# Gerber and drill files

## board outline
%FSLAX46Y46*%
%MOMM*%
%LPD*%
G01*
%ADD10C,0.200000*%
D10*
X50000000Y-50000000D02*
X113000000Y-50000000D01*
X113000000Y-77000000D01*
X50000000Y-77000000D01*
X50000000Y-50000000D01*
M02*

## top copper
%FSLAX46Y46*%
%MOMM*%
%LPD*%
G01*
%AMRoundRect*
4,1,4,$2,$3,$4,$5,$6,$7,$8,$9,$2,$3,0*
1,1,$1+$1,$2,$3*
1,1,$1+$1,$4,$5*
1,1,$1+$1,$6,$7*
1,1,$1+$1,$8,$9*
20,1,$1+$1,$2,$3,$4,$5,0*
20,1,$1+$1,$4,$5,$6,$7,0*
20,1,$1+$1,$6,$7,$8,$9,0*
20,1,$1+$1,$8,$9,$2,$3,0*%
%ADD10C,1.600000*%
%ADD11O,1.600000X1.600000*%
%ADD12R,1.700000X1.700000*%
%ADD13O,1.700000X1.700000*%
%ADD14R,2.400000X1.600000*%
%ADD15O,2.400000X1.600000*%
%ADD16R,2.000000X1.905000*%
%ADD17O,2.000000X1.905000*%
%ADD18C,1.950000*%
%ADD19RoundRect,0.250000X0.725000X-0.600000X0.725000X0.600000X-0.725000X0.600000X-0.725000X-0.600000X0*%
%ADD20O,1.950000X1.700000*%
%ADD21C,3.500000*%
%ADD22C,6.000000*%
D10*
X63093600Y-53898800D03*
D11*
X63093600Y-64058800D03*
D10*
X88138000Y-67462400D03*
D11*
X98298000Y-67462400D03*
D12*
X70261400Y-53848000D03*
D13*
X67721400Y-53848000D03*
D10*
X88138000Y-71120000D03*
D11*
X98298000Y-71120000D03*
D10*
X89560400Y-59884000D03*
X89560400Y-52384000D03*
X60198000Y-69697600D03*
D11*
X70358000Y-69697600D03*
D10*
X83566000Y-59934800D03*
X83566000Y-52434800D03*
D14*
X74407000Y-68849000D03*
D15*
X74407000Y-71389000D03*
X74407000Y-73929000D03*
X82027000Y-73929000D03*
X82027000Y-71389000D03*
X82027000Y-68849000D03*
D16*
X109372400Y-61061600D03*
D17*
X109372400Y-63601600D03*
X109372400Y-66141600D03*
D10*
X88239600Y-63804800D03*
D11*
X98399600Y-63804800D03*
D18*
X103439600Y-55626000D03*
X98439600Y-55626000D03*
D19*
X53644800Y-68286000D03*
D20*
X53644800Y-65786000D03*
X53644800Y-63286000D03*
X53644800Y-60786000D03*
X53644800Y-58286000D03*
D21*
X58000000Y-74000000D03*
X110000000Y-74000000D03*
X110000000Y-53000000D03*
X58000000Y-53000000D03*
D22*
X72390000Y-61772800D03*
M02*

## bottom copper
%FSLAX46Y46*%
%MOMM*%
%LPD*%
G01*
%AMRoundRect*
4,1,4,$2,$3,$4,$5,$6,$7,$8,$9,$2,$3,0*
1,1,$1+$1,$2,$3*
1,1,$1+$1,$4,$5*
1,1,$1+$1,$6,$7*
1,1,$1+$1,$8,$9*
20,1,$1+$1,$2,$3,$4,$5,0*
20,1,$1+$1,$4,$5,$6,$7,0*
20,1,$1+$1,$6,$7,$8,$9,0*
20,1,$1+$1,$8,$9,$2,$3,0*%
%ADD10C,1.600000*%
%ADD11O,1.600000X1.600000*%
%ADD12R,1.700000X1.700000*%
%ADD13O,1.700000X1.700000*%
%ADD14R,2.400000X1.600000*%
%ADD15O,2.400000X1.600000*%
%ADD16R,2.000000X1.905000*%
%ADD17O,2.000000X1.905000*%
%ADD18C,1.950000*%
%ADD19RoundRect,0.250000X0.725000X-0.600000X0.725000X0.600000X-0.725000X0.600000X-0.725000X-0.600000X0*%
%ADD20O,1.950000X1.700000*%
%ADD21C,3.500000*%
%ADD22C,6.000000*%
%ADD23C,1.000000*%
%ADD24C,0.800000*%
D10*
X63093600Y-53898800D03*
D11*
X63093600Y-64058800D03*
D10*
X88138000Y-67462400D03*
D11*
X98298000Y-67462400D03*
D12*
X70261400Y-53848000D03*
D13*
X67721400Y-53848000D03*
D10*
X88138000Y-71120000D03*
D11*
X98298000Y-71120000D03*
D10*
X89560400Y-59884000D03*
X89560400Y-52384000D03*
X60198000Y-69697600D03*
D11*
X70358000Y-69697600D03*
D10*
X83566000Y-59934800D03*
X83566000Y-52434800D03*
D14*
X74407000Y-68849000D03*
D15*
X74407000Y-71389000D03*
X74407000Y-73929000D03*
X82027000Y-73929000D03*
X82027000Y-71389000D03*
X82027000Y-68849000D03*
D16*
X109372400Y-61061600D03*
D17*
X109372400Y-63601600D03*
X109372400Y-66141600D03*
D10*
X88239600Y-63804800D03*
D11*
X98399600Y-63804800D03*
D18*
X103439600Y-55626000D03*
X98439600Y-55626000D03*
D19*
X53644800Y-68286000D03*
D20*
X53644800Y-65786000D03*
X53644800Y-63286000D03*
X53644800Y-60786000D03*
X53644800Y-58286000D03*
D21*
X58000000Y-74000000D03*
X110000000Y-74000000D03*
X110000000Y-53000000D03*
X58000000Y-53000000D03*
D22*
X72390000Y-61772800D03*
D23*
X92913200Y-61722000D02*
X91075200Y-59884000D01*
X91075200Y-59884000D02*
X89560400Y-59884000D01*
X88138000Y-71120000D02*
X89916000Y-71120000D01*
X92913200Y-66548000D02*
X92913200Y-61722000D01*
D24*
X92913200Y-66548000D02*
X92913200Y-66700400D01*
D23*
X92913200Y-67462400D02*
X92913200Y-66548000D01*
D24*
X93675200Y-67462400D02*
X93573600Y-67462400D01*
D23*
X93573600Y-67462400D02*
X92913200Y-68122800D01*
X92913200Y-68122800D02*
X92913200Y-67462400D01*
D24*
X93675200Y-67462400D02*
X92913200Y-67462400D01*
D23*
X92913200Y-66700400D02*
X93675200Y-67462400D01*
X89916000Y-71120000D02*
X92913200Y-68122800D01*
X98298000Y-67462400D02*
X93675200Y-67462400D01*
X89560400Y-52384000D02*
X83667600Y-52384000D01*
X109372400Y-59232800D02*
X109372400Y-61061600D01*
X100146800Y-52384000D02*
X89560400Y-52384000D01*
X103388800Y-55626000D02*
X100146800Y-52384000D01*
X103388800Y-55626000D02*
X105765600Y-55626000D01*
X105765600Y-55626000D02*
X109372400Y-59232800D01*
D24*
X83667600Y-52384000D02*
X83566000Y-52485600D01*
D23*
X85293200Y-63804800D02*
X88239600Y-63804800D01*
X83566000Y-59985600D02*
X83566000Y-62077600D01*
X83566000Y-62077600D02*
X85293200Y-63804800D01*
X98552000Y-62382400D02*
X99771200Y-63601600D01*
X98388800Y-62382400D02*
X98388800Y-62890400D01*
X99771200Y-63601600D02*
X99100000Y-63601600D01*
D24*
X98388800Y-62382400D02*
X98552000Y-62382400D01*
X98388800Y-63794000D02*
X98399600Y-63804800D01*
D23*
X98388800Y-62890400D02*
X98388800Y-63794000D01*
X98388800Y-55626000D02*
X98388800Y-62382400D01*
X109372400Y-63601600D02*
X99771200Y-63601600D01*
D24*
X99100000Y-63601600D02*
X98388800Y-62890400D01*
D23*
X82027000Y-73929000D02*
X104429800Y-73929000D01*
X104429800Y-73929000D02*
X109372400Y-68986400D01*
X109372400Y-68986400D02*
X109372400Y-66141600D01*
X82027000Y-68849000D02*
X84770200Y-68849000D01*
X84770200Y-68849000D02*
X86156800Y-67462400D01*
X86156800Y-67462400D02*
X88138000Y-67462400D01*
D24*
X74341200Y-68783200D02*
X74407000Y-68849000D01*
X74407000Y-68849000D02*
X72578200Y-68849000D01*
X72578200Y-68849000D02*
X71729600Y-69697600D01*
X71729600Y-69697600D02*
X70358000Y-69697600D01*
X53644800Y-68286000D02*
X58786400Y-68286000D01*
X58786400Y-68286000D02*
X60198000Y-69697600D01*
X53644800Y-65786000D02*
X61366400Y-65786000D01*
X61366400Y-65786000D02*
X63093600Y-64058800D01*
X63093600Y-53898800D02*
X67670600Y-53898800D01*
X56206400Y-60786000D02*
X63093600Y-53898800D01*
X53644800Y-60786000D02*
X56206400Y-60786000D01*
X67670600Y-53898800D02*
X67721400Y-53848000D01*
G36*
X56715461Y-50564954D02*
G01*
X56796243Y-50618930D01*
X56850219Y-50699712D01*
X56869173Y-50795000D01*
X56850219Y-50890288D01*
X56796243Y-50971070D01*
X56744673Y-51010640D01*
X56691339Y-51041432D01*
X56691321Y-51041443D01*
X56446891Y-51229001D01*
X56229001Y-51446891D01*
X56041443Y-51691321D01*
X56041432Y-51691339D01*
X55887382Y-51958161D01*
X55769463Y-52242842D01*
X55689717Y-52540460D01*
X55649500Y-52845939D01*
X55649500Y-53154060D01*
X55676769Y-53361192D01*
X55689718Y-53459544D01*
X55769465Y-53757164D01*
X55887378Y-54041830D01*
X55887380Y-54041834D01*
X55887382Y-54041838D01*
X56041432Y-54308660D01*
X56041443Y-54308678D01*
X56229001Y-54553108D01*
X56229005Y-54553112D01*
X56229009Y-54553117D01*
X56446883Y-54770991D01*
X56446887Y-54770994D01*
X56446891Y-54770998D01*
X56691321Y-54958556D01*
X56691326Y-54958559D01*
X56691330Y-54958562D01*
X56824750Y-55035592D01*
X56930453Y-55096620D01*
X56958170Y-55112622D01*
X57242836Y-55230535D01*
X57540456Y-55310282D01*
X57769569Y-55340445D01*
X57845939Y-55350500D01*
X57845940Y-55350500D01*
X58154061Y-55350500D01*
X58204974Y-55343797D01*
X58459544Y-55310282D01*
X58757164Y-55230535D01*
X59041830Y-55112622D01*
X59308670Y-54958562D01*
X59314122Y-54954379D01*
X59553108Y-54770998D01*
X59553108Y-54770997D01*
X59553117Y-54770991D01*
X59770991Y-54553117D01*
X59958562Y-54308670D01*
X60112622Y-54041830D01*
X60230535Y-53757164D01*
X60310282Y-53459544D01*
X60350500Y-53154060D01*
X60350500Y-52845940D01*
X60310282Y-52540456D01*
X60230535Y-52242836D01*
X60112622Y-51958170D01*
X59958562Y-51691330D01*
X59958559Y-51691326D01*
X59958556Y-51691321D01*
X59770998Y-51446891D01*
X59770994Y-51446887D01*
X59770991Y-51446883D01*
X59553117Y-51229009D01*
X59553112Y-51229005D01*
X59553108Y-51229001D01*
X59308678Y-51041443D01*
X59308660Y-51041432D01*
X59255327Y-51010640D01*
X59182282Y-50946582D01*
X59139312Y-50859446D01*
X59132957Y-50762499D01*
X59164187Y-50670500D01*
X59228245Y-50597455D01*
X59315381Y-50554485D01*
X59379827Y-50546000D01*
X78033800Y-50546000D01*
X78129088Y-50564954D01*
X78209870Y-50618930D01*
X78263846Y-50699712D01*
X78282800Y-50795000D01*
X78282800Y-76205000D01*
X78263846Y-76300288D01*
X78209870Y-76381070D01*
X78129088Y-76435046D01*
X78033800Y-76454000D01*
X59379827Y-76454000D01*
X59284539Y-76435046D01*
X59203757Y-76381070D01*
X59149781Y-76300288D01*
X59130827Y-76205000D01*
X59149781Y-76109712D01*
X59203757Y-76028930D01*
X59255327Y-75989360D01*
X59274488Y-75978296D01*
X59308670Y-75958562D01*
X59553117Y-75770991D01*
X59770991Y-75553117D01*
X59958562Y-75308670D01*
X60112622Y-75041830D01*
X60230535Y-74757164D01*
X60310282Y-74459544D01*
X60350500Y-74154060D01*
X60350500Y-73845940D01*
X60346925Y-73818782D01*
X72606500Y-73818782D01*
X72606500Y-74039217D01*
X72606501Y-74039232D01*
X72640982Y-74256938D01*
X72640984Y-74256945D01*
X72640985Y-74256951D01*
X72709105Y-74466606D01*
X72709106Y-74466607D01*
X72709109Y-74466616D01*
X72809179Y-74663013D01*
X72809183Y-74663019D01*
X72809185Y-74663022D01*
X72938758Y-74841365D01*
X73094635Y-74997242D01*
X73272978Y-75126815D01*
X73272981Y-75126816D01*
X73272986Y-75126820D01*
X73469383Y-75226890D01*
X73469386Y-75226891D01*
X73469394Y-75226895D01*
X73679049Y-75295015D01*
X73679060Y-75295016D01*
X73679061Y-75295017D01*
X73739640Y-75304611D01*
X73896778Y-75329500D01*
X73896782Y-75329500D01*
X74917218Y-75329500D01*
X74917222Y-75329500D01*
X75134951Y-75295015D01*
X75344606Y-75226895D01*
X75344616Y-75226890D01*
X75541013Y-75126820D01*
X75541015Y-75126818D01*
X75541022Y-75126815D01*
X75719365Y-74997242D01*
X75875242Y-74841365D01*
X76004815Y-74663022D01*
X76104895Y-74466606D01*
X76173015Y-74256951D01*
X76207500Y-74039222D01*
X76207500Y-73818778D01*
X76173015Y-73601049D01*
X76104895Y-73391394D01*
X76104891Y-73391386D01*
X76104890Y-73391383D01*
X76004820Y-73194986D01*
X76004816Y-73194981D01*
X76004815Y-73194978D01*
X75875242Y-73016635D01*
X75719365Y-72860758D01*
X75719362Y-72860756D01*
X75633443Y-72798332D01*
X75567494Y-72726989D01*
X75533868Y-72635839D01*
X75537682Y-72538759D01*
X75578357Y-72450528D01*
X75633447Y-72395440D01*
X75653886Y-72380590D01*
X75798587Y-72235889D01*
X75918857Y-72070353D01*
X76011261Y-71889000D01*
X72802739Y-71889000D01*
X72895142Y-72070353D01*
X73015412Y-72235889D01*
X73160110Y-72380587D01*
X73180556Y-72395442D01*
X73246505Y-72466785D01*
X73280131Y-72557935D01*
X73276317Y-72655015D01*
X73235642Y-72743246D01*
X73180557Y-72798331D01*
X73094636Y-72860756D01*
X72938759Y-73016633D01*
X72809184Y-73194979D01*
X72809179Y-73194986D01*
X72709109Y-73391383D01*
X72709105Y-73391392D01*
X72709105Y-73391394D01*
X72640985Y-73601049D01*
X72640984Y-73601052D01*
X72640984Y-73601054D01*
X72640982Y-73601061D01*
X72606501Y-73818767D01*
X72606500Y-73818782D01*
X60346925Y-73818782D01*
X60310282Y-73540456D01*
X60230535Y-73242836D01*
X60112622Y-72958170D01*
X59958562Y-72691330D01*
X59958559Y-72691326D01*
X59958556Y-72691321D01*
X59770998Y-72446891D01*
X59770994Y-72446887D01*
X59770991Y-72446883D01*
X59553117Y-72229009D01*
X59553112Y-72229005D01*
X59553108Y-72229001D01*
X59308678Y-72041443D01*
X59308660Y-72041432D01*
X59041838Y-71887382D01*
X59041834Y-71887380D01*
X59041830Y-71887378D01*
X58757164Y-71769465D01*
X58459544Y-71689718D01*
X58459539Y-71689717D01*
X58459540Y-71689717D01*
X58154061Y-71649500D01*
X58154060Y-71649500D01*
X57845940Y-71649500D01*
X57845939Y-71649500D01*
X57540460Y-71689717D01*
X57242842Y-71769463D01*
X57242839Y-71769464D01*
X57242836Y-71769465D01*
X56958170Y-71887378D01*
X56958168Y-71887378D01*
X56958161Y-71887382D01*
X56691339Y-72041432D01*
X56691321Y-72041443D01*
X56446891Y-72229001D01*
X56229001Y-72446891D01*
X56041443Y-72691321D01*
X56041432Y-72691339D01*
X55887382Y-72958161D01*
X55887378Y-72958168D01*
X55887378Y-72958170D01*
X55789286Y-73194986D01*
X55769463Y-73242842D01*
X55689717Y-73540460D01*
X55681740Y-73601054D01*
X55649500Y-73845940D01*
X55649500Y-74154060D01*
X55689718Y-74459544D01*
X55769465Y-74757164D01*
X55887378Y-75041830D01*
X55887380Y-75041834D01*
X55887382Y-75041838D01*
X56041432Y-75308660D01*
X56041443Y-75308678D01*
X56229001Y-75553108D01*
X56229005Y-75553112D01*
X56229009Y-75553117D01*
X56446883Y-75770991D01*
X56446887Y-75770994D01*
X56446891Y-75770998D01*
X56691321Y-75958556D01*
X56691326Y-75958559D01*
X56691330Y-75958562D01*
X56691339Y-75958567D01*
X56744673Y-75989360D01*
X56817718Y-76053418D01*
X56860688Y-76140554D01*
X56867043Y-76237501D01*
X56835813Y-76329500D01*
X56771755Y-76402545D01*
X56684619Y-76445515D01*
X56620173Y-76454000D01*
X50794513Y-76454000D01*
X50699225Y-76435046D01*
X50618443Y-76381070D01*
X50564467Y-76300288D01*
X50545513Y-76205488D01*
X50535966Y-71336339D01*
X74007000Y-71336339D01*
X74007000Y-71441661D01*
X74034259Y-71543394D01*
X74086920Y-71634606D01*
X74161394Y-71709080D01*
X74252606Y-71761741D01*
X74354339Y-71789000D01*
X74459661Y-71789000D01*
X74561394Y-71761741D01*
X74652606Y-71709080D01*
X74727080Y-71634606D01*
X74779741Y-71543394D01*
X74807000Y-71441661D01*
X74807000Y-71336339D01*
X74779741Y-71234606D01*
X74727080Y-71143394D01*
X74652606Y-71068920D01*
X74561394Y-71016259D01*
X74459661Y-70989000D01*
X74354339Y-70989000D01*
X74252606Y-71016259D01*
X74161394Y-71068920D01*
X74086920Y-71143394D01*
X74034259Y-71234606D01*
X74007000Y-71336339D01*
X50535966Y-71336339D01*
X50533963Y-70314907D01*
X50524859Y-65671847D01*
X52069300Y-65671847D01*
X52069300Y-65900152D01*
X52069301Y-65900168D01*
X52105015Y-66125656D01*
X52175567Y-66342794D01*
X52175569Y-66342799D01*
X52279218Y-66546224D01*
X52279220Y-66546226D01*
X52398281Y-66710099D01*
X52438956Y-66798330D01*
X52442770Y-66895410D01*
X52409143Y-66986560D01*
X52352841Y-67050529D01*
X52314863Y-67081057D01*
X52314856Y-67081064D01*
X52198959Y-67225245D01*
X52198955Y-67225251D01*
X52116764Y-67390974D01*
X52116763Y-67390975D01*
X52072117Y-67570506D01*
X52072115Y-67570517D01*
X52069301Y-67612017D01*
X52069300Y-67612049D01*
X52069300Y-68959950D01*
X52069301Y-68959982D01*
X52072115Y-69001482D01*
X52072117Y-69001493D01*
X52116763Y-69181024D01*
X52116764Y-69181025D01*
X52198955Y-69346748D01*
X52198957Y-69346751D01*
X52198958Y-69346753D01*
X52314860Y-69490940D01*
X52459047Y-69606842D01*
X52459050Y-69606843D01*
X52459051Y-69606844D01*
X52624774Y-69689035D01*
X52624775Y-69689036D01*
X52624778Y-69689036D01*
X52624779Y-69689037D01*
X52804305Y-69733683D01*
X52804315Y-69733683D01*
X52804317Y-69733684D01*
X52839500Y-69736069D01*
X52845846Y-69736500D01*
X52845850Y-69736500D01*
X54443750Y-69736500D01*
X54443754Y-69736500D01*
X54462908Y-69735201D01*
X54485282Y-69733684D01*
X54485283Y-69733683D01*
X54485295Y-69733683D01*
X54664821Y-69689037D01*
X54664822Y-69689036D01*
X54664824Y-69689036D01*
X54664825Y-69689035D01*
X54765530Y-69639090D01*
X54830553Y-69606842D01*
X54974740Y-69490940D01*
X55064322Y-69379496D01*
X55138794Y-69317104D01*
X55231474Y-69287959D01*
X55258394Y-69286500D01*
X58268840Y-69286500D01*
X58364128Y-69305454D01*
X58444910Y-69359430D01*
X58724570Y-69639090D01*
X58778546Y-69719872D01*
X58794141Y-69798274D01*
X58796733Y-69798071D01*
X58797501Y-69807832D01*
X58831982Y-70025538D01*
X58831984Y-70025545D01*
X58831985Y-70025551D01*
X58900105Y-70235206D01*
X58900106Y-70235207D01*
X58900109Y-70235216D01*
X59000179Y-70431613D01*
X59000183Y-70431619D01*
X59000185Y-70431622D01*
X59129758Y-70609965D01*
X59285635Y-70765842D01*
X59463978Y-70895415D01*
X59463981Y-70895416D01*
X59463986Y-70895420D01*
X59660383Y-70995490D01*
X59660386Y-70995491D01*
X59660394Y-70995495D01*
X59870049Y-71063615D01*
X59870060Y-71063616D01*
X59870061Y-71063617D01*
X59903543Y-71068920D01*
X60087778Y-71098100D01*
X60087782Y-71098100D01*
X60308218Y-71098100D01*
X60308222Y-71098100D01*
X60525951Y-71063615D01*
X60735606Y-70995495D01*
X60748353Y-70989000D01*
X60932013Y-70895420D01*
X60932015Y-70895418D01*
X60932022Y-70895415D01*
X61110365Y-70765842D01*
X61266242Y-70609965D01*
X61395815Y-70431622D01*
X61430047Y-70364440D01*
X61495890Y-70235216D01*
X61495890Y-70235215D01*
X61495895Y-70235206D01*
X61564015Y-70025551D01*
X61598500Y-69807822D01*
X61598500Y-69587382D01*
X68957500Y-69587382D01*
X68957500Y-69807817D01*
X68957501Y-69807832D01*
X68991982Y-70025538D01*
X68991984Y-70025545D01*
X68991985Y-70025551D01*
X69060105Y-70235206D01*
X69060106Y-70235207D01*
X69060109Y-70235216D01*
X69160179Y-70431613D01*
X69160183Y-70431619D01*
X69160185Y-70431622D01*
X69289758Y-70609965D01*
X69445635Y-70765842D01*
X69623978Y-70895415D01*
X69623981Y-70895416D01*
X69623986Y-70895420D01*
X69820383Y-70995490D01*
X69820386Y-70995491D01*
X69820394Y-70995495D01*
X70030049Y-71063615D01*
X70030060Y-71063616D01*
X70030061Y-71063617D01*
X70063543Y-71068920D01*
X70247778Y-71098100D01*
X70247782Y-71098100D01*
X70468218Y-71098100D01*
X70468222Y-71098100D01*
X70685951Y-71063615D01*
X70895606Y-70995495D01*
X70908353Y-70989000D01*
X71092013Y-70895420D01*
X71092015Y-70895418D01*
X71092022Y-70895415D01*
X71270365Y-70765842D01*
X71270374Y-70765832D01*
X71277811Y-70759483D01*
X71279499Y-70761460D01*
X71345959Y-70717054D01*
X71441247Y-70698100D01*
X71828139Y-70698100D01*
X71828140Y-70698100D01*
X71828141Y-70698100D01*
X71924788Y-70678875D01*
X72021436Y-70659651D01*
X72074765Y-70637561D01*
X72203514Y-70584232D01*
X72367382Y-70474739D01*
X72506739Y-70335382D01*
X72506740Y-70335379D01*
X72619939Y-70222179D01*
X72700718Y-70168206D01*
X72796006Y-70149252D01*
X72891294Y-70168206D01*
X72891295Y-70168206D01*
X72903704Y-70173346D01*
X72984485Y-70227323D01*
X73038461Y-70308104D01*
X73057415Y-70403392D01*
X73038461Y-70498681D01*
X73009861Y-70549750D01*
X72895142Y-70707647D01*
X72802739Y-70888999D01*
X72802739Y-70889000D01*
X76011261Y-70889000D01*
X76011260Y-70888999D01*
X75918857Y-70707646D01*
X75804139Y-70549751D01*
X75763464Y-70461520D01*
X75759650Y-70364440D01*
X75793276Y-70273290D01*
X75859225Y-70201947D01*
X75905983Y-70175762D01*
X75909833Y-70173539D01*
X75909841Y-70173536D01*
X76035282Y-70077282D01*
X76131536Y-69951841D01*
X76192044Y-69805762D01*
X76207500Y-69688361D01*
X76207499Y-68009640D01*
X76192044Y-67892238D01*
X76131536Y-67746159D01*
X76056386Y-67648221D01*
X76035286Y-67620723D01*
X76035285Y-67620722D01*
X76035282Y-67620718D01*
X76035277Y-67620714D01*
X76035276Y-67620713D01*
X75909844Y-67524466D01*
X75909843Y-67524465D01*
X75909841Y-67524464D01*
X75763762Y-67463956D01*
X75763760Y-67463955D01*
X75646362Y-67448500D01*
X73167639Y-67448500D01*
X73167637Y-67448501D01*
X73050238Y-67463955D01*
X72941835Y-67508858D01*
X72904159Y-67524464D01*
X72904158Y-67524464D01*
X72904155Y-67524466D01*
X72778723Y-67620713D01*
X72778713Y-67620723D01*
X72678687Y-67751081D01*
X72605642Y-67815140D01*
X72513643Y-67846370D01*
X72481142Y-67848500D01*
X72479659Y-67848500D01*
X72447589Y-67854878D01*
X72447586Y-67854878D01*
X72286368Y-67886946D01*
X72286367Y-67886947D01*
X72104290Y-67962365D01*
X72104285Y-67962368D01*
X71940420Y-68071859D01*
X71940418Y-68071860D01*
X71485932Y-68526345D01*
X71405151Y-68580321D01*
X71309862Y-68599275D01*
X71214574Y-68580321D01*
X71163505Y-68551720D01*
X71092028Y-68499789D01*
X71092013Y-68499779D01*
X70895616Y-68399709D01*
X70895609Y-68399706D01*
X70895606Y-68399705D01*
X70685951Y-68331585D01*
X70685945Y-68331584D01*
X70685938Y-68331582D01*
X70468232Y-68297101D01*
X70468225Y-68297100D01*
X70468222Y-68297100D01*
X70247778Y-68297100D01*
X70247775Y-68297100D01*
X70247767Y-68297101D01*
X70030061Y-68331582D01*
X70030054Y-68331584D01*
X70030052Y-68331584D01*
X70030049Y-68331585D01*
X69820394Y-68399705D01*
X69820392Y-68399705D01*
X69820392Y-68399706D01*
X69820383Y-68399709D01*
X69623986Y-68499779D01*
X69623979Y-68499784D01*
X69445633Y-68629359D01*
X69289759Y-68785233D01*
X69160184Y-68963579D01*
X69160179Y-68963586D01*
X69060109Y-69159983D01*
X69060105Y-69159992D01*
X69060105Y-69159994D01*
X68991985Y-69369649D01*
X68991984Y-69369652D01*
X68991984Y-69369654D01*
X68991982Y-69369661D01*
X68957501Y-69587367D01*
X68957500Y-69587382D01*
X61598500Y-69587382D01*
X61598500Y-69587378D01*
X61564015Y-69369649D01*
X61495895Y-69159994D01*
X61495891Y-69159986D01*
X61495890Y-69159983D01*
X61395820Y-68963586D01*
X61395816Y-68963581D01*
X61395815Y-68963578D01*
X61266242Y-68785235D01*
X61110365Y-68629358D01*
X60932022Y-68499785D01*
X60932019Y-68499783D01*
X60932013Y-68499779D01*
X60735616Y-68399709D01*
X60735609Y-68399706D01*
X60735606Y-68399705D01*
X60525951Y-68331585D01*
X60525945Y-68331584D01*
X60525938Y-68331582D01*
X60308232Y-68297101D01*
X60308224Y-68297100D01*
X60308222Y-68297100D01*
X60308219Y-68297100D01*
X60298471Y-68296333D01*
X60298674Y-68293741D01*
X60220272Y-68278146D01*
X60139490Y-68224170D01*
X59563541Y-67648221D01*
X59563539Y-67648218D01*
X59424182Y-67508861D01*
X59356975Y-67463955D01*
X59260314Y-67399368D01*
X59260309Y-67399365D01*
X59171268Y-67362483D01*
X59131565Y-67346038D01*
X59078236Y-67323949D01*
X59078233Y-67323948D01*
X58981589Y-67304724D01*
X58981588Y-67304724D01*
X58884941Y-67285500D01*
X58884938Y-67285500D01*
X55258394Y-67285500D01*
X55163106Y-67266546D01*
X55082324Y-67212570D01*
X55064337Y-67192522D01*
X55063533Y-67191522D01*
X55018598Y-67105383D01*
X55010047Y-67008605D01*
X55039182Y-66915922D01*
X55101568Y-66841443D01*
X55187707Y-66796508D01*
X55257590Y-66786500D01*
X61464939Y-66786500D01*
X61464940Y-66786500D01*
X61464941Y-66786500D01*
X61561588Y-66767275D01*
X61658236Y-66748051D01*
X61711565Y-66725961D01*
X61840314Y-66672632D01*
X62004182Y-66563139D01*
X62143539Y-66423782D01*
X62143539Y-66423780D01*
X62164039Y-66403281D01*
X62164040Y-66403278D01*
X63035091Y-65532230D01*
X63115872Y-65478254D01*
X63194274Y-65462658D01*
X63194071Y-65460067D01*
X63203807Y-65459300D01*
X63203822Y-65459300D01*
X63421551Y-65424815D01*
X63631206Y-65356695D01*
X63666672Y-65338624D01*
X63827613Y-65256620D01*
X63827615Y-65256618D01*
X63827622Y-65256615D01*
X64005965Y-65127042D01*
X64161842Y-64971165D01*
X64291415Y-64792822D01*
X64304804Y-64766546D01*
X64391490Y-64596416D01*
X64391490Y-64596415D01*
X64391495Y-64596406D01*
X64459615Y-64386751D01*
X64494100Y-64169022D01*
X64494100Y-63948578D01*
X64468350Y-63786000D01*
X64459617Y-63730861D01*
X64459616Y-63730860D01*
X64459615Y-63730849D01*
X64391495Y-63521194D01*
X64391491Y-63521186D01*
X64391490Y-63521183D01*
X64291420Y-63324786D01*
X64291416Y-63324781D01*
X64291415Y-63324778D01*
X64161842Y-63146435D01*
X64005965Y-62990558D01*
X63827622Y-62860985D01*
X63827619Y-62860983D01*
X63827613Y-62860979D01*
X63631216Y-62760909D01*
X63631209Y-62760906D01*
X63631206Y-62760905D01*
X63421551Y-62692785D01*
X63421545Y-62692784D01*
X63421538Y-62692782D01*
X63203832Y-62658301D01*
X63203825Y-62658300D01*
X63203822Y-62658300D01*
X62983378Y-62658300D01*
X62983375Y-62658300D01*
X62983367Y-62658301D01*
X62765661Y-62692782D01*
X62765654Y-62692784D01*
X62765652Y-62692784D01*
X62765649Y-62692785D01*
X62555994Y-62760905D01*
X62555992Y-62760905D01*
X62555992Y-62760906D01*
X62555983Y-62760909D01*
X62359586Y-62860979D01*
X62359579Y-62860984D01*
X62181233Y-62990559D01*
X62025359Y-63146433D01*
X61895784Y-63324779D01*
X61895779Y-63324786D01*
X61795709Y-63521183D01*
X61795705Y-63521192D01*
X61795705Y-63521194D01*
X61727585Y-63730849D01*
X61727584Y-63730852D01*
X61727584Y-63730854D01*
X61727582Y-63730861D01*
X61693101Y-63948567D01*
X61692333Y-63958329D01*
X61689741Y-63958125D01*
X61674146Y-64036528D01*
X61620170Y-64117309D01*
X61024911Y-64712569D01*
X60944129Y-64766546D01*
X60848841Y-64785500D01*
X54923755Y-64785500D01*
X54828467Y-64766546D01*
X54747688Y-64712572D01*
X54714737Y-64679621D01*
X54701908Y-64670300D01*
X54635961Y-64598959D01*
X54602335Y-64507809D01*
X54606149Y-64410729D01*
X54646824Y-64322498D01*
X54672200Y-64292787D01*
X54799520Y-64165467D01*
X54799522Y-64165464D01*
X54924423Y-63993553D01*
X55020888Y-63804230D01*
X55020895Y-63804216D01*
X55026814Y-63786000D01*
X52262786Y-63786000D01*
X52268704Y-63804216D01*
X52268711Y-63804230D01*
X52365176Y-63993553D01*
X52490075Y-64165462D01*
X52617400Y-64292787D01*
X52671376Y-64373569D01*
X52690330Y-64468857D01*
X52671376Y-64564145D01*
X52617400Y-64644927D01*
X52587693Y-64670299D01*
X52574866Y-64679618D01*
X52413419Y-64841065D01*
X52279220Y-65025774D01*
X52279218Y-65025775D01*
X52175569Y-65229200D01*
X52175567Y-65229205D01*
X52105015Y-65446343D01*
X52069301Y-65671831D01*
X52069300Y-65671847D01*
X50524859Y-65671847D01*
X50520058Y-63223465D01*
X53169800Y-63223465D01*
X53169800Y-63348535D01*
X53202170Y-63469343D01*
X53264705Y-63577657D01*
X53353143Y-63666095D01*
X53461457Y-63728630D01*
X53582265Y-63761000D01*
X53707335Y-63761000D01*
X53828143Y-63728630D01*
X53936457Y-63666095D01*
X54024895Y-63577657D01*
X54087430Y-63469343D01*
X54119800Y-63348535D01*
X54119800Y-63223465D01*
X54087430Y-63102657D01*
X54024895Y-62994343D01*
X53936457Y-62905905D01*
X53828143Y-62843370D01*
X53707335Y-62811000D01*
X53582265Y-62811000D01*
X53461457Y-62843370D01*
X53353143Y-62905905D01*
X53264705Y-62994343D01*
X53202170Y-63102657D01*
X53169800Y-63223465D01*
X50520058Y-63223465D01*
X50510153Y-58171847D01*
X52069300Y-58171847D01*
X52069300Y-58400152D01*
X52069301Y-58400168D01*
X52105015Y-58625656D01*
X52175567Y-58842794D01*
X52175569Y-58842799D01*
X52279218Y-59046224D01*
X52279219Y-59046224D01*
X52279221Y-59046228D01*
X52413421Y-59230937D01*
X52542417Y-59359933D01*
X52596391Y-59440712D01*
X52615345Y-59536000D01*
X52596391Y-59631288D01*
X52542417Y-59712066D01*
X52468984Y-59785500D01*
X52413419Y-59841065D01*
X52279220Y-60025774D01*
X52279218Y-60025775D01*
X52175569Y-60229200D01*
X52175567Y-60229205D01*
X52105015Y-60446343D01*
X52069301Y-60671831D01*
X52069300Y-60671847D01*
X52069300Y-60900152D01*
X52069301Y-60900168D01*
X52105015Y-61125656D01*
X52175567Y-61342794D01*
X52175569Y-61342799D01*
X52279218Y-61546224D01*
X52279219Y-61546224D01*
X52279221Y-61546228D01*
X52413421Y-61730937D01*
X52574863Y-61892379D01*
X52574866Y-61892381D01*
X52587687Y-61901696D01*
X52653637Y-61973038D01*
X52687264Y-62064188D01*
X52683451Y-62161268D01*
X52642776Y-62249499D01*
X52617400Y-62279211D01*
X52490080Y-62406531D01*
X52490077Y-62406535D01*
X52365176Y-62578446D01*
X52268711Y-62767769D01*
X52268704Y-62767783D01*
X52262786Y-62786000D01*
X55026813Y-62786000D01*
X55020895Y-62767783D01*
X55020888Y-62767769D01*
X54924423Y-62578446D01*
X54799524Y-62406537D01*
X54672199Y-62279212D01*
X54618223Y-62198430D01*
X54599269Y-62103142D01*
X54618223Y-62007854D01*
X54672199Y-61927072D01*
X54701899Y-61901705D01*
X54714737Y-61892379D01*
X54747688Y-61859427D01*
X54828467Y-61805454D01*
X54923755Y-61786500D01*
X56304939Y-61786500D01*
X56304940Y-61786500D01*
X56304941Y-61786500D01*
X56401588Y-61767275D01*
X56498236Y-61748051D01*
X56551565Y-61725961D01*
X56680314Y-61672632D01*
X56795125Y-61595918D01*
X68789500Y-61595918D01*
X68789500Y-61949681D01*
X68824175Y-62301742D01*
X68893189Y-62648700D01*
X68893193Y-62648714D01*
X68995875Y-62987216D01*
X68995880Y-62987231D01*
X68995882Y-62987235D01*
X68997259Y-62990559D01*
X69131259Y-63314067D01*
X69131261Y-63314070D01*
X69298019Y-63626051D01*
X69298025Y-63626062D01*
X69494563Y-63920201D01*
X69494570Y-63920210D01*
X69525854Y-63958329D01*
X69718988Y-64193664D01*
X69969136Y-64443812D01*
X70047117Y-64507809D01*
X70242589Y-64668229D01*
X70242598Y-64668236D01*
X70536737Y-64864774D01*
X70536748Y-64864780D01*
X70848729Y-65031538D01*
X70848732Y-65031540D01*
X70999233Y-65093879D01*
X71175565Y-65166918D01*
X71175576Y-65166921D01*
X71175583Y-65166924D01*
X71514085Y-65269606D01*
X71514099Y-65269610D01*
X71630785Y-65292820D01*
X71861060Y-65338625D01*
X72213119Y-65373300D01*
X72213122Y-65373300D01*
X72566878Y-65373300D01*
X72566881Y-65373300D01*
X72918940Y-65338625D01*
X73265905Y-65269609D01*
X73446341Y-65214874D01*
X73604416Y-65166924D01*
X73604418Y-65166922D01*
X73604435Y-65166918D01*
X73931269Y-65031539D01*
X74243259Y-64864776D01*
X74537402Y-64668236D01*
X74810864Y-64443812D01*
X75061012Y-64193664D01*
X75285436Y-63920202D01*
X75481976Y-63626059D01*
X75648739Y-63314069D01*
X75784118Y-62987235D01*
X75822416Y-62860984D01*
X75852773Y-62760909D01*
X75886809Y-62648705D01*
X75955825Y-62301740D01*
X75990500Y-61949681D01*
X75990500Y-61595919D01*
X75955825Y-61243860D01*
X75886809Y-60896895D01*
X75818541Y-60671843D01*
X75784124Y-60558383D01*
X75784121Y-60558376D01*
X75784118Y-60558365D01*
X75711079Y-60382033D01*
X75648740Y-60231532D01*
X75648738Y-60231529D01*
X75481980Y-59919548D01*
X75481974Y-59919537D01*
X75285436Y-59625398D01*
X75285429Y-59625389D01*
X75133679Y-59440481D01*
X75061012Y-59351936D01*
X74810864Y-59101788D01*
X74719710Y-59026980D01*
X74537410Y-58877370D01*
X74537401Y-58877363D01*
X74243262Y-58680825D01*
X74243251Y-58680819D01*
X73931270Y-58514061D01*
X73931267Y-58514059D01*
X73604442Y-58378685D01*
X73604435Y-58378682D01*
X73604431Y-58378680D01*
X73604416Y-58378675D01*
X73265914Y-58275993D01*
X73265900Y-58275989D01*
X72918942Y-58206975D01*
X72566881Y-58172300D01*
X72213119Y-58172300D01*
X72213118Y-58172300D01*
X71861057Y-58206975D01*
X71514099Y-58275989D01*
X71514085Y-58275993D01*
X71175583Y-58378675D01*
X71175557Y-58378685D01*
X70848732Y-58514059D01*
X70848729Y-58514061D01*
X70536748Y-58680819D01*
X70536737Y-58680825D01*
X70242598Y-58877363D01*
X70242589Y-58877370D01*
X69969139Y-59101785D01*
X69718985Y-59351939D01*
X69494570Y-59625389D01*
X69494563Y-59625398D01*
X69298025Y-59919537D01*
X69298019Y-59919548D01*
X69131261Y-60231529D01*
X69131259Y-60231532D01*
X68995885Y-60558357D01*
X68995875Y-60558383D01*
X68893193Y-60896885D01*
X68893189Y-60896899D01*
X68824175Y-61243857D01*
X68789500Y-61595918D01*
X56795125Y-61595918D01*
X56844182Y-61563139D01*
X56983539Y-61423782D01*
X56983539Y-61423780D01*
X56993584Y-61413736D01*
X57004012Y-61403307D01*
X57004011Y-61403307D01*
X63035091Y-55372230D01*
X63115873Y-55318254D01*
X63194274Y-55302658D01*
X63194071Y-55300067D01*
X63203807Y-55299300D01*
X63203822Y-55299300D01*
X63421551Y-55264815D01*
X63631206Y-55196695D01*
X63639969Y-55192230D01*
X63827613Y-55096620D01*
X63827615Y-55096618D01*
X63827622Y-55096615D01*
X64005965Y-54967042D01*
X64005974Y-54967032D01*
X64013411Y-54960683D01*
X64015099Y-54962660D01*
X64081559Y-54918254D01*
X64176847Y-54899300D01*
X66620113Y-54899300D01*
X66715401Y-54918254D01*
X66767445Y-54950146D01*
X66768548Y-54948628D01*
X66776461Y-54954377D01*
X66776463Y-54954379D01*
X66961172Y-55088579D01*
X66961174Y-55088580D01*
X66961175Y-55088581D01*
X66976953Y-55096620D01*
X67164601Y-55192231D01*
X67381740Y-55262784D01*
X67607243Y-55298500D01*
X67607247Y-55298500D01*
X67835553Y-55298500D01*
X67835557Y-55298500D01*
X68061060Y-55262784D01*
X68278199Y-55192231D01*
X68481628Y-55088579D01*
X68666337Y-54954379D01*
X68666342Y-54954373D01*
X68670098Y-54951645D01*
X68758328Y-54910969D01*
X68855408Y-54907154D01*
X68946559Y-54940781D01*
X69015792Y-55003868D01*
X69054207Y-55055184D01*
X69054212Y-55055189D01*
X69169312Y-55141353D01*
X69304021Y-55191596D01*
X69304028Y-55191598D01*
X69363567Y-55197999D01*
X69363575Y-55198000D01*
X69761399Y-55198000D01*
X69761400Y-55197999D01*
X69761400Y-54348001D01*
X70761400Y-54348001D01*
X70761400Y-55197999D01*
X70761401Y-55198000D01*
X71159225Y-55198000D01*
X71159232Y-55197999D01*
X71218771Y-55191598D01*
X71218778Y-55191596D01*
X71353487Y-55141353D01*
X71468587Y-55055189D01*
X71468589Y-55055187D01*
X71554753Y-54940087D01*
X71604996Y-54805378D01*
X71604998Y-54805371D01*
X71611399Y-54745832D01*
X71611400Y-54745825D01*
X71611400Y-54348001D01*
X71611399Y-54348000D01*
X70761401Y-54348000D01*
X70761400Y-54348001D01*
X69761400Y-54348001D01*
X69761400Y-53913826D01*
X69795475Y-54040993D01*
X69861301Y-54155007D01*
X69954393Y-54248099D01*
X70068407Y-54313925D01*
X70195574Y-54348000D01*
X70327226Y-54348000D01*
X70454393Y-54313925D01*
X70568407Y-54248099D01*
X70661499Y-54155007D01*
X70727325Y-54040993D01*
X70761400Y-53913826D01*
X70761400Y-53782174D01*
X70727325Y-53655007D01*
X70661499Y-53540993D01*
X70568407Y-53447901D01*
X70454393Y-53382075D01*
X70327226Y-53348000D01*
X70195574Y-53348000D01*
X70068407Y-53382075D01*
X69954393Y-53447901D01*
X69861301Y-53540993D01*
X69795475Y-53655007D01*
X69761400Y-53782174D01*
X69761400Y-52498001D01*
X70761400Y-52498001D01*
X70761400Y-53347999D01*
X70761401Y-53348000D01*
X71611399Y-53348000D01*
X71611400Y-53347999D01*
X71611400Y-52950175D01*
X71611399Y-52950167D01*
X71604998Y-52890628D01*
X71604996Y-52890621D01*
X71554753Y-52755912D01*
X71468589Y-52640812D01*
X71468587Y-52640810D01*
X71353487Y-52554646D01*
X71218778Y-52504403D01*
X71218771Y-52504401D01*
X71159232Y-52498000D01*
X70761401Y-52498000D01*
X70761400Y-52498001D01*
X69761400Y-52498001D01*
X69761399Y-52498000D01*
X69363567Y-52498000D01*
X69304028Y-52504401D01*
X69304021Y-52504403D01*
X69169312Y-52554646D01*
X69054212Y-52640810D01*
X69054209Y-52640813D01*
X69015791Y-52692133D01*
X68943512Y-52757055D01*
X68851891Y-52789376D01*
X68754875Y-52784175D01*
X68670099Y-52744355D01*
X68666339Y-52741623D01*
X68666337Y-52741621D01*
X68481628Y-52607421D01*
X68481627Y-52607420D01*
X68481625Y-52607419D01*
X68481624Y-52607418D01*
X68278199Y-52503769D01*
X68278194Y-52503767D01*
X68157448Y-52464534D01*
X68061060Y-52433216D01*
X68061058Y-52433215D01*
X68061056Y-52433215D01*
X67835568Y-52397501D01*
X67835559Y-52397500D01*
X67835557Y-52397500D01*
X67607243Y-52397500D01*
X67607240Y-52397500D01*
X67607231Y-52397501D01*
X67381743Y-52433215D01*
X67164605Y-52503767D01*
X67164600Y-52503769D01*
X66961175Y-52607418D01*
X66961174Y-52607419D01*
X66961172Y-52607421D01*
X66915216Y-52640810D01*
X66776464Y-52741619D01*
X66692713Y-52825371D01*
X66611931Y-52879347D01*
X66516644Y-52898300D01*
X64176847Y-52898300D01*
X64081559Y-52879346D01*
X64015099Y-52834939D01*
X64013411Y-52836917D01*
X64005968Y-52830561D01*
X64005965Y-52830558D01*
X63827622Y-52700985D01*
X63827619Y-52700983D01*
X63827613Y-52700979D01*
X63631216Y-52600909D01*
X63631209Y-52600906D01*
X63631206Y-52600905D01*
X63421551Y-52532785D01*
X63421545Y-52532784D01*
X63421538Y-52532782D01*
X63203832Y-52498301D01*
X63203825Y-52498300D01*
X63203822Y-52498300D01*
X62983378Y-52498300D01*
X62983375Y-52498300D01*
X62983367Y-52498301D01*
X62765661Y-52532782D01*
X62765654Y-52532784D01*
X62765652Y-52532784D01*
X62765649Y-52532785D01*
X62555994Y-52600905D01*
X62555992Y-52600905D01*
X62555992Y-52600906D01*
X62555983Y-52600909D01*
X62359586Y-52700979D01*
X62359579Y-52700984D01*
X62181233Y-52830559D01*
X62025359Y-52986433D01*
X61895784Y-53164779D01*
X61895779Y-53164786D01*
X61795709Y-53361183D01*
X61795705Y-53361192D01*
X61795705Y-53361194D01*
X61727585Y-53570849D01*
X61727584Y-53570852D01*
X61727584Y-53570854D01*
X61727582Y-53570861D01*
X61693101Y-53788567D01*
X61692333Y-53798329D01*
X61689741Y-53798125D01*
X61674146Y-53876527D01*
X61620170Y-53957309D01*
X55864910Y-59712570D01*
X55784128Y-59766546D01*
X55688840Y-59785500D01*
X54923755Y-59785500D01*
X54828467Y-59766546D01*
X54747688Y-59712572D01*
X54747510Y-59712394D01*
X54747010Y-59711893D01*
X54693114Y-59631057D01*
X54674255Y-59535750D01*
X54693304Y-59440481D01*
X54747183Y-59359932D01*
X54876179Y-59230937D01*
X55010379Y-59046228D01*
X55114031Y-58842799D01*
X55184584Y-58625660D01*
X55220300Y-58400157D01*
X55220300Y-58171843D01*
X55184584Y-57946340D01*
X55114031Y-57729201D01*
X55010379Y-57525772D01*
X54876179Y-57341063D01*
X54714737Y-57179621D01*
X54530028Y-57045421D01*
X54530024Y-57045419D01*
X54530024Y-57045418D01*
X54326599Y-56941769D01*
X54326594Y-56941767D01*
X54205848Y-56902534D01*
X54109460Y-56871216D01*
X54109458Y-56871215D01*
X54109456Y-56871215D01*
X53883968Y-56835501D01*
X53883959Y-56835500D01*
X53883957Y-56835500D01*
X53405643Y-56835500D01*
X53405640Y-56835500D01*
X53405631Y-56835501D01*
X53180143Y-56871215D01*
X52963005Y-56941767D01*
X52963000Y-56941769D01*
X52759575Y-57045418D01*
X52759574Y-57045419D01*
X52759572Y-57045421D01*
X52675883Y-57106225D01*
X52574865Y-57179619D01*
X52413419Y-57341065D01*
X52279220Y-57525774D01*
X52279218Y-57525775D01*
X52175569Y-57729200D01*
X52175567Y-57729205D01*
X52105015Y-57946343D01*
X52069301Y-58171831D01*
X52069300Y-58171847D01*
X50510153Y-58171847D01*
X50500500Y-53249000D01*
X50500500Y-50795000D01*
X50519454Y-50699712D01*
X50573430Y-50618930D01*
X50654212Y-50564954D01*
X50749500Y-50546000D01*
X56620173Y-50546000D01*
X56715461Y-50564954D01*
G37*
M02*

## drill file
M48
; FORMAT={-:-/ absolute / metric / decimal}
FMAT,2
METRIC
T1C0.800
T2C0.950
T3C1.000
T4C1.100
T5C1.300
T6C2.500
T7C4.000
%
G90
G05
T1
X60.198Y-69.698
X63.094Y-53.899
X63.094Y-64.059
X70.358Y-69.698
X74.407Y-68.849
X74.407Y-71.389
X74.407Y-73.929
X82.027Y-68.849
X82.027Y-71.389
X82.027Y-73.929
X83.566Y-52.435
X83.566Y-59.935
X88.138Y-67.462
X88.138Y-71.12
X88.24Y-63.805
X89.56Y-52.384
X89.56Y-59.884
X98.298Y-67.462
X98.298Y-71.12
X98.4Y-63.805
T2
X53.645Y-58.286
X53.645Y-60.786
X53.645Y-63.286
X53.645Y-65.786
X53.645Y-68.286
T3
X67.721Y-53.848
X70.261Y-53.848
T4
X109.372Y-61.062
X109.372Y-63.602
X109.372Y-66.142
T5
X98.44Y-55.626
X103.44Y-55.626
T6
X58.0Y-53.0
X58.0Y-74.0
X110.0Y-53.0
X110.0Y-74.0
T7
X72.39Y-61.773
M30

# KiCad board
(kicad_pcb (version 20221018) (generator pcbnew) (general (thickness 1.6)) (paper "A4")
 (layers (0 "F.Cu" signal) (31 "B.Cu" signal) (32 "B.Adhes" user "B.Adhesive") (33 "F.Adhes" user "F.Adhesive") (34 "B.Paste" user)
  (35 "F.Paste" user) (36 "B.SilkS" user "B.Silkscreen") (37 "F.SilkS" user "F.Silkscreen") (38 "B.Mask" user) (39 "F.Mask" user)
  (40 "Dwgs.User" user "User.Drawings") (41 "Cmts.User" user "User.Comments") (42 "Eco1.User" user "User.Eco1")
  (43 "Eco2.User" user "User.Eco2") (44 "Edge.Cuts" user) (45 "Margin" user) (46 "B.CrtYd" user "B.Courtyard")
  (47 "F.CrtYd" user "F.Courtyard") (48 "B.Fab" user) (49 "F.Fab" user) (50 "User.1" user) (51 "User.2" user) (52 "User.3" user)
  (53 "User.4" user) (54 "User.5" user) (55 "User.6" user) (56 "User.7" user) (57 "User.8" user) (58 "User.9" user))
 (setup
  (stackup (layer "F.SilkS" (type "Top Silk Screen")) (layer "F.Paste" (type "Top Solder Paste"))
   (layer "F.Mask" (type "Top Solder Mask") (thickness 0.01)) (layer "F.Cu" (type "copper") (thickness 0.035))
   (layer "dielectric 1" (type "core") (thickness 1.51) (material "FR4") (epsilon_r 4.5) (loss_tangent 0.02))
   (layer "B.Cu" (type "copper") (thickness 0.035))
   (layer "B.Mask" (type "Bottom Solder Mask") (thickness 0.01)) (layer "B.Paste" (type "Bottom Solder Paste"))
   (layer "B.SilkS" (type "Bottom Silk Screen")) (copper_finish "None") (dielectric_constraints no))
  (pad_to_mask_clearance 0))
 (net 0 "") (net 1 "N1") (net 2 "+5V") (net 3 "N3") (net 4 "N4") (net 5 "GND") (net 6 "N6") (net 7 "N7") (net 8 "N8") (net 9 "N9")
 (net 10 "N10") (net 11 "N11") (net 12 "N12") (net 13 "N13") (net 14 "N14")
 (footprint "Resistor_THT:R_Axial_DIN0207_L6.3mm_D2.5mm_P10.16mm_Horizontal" (layer "F.Cu") (at 63.0936 53.8988 -90)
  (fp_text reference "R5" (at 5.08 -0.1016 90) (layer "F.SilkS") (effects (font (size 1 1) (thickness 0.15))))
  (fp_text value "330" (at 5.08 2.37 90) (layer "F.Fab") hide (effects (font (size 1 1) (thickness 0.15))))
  (pad "1" thru_hole circle (at 0 0 270) (size 1.6 1.6) (drill 0.8) (layers "*.Cu" "*.Mask") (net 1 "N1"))
  (pad "2" thru_hole oval (at 10.16 0 270) (size 1.6 1.6) (drill 0.8) (layers "*.Cu" "*.Mask") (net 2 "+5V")))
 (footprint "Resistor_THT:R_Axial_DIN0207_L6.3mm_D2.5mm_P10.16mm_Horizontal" (layer "F.Cu") (at 88.138 67.4624)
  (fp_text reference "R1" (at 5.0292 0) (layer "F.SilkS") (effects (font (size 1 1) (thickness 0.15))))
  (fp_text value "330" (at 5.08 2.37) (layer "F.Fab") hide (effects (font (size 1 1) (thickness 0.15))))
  (pad "1" thru_hole circle (at 0 0) (size 1.6 1.6) (drill 0.8) (layers "*.Cu" "*.Mask") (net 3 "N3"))
  (pad "2" thru_hole oval (at 10.16 0) (size 1.6 1.6) (drill 0.8) (layers "*.Cu" "*.Mask") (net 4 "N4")))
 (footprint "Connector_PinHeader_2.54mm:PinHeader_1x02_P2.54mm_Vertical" (layer "F.Cu") (at 70.2614 53.848 -90)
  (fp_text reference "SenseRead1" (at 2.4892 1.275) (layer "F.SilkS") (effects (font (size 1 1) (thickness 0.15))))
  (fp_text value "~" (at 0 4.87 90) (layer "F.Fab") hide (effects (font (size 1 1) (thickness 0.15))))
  (pad "1" thru_hole rect (at 0 0 270) (size 1.7 1.7) (drill 1) (layers "*.Cu" "*.Mask") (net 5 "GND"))
  (pad "2" thru_hole oval (at 0 2.54 270) (size 1.7 1.7) (drill 1) (layers "*.Cu" "*.Mask") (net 1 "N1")))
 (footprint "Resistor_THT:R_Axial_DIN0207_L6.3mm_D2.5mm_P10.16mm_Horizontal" (layer "F.Cu") (at 88.138 71.12)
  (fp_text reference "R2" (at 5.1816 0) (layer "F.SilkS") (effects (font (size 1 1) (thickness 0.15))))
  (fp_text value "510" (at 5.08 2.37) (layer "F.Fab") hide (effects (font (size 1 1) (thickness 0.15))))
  (pad "1" thru_hole circle (at 0 0) (size 1.6 1.6) (drill 0.8) (layers "*.Cu" "*.Mask") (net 4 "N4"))
  (pad "2" thru_hole oval (at 10.16 0) (size 1.6 1.6) (drill 0.8) (layers "*.Cu" "*.Mask") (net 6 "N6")))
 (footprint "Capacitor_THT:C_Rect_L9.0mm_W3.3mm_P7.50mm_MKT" (layer "F.Cu") (at 89.5604 59.884 90)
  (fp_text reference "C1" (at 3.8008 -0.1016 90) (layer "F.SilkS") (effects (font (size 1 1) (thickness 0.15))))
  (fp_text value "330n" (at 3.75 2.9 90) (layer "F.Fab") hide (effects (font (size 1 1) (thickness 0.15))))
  (pad "1" thru_hole circle (at 0 0 90) (size 1.6 1.6) (drill 0.8) (layers "*.Cu" "*.Mask") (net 4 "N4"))
  (pad "2" thru_hole circle (at 7.5 0 90) (size 1.6 1.6) (drill 0.8) (layers "*.Cu" "*.Mask") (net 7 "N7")))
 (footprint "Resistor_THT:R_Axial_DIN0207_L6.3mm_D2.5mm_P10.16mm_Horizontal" (layer "F.Cu") (at 60.198 69.6976)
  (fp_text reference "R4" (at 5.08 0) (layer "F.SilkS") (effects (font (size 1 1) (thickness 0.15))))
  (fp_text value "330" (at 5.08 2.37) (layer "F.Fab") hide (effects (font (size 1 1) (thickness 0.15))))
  (pad "1" thru_hole circle (at 0 0) (size 1.6 1.6) (drill 0.8) (layers "*.Cu" "*.Mask") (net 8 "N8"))
  (pad "2" thru_hole oval (at 10.16 0) (size 1.6 1.6) (drill 0.8) (layers "*.Cu" "*.Mask") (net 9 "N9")))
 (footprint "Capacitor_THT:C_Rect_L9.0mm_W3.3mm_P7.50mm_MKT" (layer "F.Cu") (at 83.566 59.9348 90)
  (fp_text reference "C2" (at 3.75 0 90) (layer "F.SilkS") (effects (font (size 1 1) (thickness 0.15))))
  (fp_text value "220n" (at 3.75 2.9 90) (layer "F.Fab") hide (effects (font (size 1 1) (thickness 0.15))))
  (pad "1" thru_hole circle (at 0 0 90) (size 1.6 1.6) (drill 0.8) (layers "*.Cu" "*.Mask") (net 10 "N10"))
  (pad "2" thru_hole circle (at 7.5 0 90) (size 1.6 1.6) (drill 0.8) (layers "*.Cu" "*.Mask") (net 7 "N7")))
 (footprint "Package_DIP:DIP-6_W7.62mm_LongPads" (layer "F.Cu") (at 74.407 68.849)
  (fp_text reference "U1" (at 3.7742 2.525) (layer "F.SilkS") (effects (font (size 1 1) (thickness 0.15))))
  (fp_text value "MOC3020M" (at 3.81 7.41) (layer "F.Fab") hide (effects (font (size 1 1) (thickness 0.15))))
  (pad "1" thru_hole rect (at 0 0) (size 2.4 1.6) (drill 0.8) (layers "*.Cu" "*.Mask") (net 9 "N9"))
  (pad "2" thru_hole oval (at 0 2.54) (size 2.4 1.6) (drill 0.8) (layers "*.Cu" "*.Mask") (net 5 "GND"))
  (pad "3" thru_hole oval (at 0 5.08) (size 2.4 1.6) (drill 0.8) (layers "*.Cu" "*.Mask") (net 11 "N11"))
  (pad "4" thru_hole oval (at 7.62 5.08) (size 2.4 1.6) (drill 0.8) (layers "*.Cu" "*.Mask") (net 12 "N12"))
  (pad "5" thru_hole oval (at 7.62 2.54) (size 2.4 1.6) (drill 0.8) (layers "*.Cu" "*.Mask") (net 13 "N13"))
  (pad "6" thru_hole oval (at 7.62 0) (size 2.4 1.6) (drill 0.8) (layers "*.Cu" "*.Mask") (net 3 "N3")))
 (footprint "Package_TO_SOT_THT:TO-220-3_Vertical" (layer "F.Cu") (at 109.3724 61.0616 -90)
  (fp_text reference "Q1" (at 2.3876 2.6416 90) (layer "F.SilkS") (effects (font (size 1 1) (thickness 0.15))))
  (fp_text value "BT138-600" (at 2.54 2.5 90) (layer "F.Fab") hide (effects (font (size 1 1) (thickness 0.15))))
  (pad "1" thru_hole rect (at 0 0 270) (size 1.905 2) (drill 1.1) (layers "*.Cu" "*.Mask") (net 7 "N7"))
  (pad "2" thru_hole oval (at 2.54 0 270) (size 1.905 2) (drill 1.1) (layers "*.Cu" "*.Mask") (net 6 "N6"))
  (pad "3" thru_hole oval (at 5.08 0 270) (size 1.905 2) (drill 1.1) (layers "*.Cu" "*.Mask") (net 12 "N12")))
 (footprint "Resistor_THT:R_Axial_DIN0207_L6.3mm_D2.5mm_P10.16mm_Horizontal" (layer "F.Cu") (at 88.2396 63.8048)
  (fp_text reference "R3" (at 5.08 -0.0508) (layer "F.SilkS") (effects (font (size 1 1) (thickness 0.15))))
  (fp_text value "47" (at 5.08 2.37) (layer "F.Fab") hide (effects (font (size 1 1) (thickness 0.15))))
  (pad "1" thru_hole circle (at 0 0) (size 1.6 1.6) (drill 0.8) (layers "*.Cu" "*.Mask") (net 10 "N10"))
  (pad "2" thru_hole oval (at 10.16 0) (size 1.6 1.6) (drill 0.8) (layers "*.Cu" "*.Mask") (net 6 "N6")))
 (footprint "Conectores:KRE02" (layer "F.Cu") (at 103.4396 55.626 180)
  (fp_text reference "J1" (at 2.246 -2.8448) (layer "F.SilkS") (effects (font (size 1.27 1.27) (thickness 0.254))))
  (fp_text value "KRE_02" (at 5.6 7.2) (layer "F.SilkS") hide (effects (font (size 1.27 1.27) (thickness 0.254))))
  (pad "1" thru_hole circle (at 0 0 180) (size 1.95 1.95) (drill 1.3) (layers "*.Cu" "*.Mask") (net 7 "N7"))
  (pad "2" thru_hole circle (at 5 0 180) (size 1.95 1.95) (drill 1.3) (layers "*.Cu" "*.Mask") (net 6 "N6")))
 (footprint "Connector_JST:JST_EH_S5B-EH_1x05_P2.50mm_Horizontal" (layer "F.Cu") (at 53.6448 68.286 90)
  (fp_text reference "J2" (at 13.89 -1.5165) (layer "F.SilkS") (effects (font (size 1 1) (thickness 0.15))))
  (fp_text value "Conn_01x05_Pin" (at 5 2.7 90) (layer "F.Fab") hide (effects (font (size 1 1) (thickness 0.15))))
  (pad "1" thru_hole roundrect (at 0 0 90) (size 1.7 1.95) (drill 0.95) (layers "*.Cu" "*.Mask") (roundrect_rratio 0.147059) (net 8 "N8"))
  (pad "2" thru_hole oval (at 2.5 0 90) (size 1.7 1.95) (drill 0.95) (layers "*.Cu" "*.Mask") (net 2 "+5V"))
  (pad "3" thru_hole oval (at 5 0 90) (size 1.7 1.95) (drill 0.95) (layers "*.Cu" "*.Mask") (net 5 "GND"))
  (pad "4" thru_hole oval (at 7.5 0 90) (size 1.7 1.95) (drill 0.95) (layers "*.Cu" "*.Mask") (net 1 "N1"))
  (pad "5" thru_hole oval (at 10 0 90) (size 1.7 1.95) (drill 0.95) (layers "*.Cu" "*.Mask") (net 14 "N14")))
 (gr_rect (start 50 50) (end 113 77) (stroke (width 0.2) (type default)) (fill none) (layer "Edge.Cuts"))
 (via (at 58 74) (size 3.5) (drill 2.5) (layers "F.Cu" "B.Cu") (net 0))
 (via (at 110 74) (size 3.5) (drill 2.5) (layers "F.Cu" "B.Cu") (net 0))
 (via (at 110 53) (size 3.5) (drill 2.5) (layers "F.Cu" "B.Cu") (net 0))
 (via (at 58 53) (size 3.5) (drill 2.5) (layers "F.Cu" "B.Cu") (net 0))
 (via (at 72.39 61.7728) (size 6) (drill 4) (layers "F.Cu" "B.Cu") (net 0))
 (segment (start 92.9132 61.722) (end 91.0752 59.884) (width 1) (layer "B.Cu") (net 4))
 (segment (start 91.0752 59.884) (end 89.5604 59.884) (width 1) (layer "B.Cu") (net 4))
 (segment (start 88.138 71.12) (end 89.916 71.12) (width 1) (layer "B.Cu") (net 4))
 (segment (start 92.9132 66.548) (end 92.9132 61.722) (width 1) (layer "B.Cu") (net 4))
 (segment (start 92.9132 66.548) (end 92.9132 66.7004) (width 0.8) (layer "B.Cu") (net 4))
 (segment (start 92.9132 67.4624) (end 92.9132 66.548) (width 1) (layer "B.Cu") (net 4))
 (segment (start 93.6752 67.4624) (end 93.5736 67.4624) (width 0.8) (layer "B.Cu") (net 4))
 (segment (start 93.5736 67.4624) (end 92.9132 68.1228) (width 1) (layer "B.Cu") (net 4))
 (segment (start 92.9132 68.1228) (end 92.9132 67.4624) (width 1) (layer "B.Cu") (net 4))
 (segment (start 93.6752 67.4624) (end 92.9132 67.4624) (width 0.8) (layer "B.Cu") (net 4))
 (segment (start 92.9132 66.7004) (end 93.6752 67.4624) (width 1) (layer "B.Cu") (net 4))
 (segment (start 89.916 71.12) (end 92.9132 68.1228) (width 1) (layer "B.Cu") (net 4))
 (segment (start 98.298 67.4624) (end 93.6752 67.4624) (width 1) (layer "B.Cu") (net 4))
 (segment (start 89.5604 52.384) (end 83.6676 52.384) (width 1) (layer "B.Cu") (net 7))
 (segment (start 109.3724 59.2328) (end 109.3724 61.0616) (width 1) (layer "B.Cu") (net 7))
 (segment (start 100.1468 52.384) (end 89.5604 52.384) (width 1) (layer "B.Cu") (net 7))
 (segment (start 103.3888 55.626) (end 100.1468 52.384) (width 1) (layer "B.Cu") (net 7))
 (segment (start 103.3888 55.626) (end 105.7656 55.626) (width 1) (layer "B.Cu") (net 7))
 (segment (start 105.7656 55.626) (end 109.3724 59.2328) (width 1) (layer "B.Cu") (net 7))
 (segment (start 83.6676 52.384) (end 83.566 52.4856) (width 0.8) (layer "B.Cu") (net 7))
 (segment (start 85.2932 63.8048) (end 88.2396 63.8048) (width 1) (layer "B.Cu") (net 10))
 (segment (start 83.566 59.9856) (end 83.566 62.0776) (width 1) (layer "B.Cu") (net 10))
 (segment (start 83.566 62.0776) (end 85.2932 63.8048) (width 1) (layer "B.Cu") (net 10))
 (segment (start 98.552 62.3824) (end 99.7712 63.6016) (width 1) (layer "B.Cu") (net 6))
 (segment (start 98.3888 62.3824) (end 98.3888 62.8904) (width 1) (layer "B.Cu") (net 6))
 (segment (start 99.7712 63.6016) (end 99.1 63.6016) (width 1) (layer "B.Cu") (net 6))
 (segment (start 98.3888 62.3824) (end 98.552 62.3824) (width 0.8) (layer "B.Cu") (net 6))
 (segment (start 98.3888 63.794) (end 98.3996 63.8048) (width 0.8) (layer "B.Cu") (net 6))
 (segment (start 98.3888 62.8904) (end 98.3888 63.794) (width 1) (layer "B.Cu") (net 6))
 (segment (start 98.3888 55.626) (end 98.3888 62.3824) (width 1) (layer "B.Cu") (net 6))
 (segment (start 109.3724 63.6016) (end 99.7712 63.6016) (width 1) (layer "B.Cu") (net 6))
 (segment (start 99.1 63.6016) (end 98.3888 62.8904) (width 0.8) (layer "B.Cu") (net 6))
 (segment (start 82.027 73.929) (end 104.4298 73.929) (width 1) (layer "B.Cu") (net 12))
 (segment (start 104.4298 73.929) (end 109.3724 68.9864) (width 1) (layer "B.Cu") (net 12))
 (segment (start 109.3724 68.9864) (end 109.3724 66.1416) (width 1) (layer "B.Cu") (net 12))
 (segment (start 82.027 68.849) (end 84.7702 68.849) (width 1) (layer "B.Cu") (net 3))
 (segment (start 84.7702 68.849) (end 86.1568 67.4624) (width 1) (layer "B.Cu") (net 3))
 (segment (start 86.1568 67.4624) (end 88.138 67.4624) (width 1) (layer "B.Cu") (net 3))
 (segment (start 74.3412 68.7832) (end 74.407 68.849) (width 0.8) (layer "B.Cu") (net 9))
 (segment (start 74.407 68.849) (end 72.5782 68.849) (width 0.8) (layer "B.Cu") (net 9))
 (segment (start 72.5782 68.849) (end 71.7296 69.6976) (width 0.8) (layer "B.Cu") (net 9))
 (segment (start 71.7296 69.6976) (end 70.358 69.6976) (width 0.8) (layer "B.Cu") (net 9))
 (segment (start 53.6448 68.286) (end 58.7864 68.286) (width 0.8) (layer "B.Cu") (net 8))
 (segment (start 58.7864 68.286) (end 60.198 69.6976) (width 0.8) (layer "B.Cu") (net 8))
 (segment (start 53.6448 65.786) (end 61.3664 65.786) (width 0.8) (layer "B.Cu") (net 2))
 (segment (start 61.3664 65.786) (end 63.0936 64.0588) (width 0.8) (layer "B.Cu") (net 2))
 (segment (start 63.0936 53.8988) (end 67.6706 53.8988) (width 0.8) (layer "B.Cu") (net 1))
 (segment (start 56.2064 60.786) (end 63.0936 53.8988) (width 0.8) (layer "B.Cu") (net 1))
 (segment (start 53.6448 60.786) (end 56.2064 60.786) (width 0.8) (layer "B.Cu") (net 1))
 (segment (start 67.6706 53.8988) (end 67.7214 53.848) (width 0.8) (layer "B.Cu") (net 1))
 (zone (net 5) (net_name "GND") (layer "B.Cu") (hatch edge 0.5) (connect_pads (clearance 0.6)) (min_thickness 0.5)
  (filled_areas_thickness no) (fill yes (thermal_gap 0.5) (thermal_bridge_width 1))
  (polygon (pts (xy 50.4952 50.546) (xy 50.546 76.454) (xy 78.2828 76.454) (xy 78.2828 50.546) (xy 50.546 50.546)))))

